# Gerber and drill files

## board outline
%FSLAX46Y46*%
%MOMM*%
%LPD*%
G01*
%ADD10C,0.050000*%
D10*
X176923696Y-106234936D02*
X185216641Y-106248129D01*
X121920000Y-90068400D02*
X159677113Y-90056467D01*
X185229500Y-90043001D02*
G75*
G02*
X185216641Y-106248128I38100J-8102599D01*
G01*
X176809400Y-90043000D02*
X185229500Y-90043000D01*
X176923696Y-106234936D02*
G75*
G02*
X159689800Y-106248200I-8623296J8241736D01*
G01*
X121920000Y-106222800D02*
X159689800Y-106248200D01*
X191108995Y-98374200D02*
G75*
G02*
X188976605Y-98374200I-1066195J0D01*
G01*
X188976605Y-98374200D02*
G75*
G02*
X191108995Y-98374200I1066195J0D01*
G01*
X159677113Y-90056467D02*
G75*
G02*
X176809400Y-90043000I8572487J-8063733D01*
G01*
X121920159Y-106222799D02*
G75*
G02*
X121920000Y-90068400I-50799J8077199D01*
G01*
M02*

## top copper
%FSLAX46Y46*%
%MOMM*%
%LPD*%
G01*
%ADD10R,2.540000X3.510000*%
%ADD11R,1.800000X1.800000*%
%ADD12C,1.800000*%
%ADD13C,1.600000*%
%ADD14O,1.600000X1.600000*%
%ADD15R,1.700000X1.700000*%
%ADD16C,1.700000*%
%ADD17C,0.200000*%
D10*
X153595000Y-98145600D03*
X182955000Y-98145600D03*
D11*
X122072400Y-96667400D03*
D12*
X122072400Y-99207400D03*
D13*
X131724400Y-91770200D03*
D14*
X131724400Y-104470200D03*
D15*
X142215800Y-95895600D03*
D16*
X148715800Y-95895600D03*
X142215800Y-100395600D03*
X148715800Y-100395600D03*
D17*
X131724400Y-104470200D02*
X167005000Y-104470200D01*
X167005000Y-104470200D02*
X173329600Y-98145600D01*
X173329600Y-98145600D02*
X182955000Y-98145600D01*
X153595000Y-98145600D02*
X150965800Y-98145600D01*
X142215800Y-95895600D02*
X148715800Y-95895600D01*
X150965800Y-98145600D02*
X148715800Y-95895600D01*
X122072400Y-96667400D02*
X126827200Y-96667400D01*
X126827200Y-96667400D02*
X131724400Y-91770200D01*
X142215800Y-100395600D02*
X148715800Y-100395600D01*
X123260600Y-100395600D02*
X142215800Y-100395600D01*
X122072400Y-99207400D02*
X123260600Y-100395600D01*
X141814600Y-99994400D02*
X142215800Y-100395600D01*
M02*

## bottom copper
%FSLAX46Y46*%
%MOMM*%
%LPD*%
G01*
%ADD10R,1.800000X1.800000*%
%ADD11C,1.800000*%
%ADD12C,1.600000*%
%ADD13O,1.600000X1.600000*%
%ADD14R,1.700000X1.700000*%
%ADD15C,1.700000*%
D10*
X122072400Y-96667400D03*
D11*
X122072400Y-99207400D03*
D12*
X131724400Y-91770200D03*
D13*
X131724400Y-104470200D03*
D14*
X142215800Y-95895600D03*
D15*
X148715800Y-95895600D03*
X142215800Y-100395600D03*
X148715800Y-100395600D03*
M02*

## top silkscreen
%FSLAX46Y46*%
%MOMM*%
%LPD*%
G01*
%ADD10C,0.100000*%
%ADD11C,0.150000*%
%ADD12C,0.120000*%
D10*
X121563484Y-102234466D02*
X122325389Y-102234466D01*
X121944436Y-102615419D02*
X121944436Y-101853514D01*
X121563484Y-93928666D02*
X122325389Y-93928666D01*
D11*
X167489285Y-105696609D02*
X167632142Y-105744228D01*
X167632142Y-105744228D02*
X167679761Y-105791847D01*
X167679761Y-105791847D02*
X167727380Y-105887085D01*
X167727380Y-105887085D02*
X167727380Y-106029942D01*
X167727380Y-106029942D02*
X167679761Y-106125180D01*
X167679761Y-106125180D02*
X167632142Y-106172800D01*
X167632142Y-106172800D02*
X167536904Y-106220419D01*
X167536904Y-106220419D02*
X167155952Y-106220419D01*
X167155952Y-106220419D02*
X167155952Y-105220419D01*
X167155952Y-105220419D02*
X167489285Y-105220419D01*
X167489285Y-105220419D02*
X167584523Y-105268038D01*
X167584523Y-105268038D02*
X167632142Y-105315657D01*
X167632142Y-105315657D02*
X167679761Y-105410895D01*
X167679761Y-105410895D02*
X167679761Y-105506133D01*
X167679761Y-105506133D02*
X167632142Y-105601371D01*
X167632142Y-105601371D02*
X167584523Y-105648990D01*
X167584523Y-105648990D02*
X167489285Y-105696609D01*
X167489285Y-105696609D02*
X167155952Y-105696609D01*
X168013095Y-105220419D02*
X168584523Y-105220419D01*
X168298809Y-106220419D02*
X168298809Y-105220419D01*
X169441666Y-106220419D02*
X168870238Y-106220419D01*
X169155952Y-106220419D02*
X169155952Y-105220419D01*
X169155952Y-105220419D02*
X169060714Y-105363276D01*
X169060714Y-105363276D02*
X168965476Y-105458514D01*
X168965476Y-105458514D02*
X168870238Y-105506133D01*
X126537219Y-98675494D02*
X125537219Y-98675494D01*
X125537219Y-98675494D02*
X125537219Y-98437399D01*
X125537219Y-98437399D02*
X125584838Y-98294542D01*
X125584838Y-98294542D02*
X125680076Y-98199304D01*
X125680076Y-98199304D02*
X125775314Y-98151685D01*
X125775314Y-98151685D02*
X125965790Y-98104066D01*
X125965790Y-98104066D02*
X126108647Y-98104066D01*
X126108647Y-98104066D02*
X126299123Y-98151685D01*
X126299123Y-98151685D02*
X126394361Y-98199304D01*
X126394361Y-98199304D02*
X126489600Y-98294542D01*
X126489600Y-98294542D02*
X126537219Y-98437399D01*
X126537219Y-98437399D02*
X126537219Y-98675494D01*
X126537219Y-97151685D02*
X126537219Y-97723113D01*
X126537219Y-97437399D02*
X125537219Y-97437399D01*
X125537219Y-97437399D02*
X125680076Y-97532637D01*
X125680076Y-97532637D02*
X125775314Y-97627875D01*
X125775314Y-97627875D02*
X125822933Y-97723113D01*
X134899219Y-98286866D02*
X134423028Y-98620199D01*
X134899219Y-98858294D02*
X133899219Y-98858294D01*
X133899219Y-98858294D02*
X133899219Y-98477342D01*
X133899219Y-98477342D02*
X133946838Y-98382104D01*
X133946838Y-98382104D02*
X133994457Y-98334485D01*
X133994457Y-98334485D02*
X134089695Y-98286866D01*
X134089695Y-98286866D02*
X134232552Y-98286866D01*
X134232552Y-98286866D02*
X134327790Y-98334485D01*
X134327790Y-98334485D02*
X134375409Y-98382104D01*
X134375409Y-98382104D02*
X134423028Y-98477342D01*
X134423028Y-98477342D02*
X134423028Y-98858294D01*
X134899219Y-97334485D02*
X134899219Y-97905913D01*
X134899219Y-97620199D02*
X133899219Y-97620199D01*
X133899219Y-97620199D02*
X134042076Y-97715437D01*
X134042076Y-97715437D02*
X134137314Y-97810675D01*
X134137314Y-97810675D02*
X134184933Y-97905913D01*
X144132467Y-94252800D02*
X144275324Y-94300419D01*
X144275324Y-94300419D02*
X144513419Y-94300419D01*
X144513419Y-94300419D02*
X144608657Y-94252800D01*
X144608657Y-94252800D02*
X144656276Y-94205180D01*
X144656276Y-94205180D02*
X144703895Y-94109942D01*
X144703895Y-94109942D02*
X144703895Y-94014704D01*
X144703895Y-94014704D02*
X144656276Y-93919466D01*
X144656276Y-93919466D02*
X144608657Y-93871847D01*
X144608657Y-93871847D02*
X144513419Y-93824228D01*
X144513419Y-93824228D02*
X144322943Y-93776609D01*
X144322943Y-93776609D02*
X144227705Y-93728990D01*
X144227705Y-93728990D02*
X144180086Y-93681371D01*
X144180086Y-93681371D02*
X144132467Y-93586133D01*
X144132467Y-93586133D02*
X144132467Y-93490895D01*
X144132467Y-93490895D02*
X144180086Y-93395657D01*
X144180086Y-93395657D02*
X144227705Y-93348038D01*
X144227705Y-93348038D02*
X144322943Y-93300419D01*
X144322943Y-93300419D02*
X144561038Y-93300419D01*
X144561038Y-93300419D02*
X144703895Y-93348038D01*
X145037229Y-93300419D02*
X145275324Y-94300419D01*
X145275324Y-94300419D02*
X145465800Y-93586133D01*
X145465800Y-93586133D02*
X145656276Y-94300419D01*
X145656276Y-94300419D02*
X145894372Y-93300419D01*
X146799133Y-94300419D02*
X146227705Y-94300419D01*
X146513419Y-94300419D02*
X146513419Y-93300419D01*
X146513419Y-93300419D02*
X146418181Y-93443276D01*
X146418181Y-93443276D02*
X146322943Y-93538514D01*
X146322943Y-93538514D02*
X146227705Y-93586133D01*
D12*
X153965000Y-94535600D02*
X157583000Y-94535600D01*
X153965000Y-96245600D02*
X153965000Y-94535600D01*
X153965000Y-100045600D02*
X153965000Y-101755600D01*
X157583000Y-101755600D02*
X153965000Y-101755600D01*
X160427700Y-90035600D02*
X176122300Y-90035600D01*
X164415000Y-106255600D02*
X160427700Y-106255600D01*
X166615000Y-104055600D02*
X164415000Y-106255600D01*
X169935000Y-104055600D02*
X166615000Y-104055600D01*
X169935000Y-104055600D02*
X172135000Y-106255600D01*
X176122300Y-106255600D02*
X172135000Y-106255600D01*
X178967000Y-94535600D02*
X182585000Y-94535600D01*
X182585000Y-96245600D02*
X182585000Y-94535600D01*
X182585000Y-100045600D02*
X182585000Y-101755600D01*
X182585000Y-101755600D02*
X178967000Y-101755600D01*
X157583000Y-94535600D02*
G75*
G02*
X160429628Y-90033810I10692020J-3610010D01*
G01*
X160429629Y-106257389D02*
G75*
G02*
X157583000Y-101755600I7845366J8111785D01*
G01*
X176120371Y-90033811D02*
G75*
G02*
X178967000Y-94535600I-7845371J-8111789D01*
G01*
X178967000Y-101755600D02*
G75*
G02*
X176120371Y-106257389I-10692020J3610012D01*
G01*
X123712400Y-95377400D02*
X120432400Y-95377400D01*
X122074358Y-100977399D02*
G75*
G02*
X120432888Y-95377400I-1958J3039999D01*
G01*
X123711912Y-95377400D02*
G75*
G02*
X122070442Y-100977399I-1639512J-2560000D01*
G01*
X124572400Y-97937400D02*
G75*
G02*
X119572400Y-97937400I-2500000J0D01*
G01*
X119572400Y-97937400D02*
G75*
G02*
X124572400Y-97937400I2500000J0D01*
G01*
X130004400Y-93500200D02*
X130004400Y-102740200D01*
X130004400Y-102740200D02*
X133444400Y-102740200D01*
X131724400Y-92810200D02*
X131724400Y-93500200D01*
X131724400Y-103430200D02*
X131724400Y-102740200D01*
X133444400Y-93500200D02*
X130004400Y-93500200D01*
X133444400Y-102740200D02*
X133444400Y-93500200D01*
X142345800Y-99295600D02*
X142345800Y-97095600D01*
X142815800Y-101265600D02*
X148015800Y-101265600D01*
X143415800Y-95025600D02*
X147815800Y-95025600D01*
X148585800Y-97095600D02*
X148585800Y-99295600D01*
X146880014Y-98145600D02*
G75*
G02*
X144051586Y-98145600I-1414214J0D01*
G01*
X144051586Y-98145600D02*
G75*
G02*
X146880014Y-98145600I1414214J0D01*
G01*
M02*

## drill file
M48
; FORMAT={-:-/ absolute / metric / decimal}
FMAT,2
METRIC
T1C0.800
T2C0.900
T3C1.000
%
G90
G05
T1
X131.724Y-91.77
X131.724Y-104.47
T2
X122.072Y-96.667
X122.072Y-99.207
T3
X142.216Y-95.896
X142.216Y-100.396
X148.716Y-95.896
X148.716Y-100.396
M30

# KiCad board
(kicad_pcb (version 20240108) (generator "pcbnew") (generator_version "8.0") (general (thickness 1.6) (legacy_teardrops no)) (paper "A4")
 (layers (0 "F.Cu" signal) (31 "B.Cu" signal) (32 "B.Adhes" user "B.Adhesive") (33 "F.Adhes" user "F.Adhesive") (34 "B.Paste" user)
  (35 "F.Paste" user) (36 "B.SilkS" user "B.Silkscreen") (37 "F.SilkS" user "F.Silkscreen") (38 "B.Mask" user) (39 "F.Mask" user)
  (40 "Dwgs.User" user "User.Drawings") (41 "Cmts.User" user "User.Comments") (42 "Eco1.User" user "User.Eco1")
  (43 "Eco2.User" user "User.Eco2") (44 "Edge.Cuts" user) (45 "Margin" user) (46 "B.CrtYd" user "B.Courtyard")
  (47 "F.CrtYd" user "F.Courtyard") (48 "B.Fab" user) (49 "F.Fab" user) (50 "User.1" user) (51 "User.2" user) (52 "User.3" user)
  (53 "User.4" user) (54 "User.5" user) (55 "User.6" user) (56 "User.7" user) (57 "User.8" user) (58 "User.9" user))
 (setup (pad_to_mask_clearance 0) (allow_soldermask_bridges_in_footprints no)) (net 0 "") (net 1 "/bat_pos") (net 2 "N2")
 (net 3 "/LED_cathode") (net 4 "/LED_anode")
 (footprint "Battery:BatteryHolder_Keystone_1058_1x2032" (layer "F.Cu") (at 168.275 98.1456)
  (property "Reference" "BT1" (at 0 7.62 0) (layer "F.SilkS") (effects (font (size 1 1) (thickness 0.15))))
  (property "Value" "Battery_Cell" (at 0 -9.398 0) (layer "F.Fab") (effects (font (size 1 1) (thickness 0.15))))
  (fp_line (start -14.31 -3.61) (end -10.692 -3.61) (stroke (width 0.12) (type solid)) (layer "F.SilkS"))
  (fp_line (start -14.31 -1.9) (end -14.31 -3.61) (stroke (width 0.12) (type solid)) (layer "F.SilkS"))
  (fp_line (start -14.31 1.9) (end -14.31 3.61) (stroke (width 0.12) (type solid)) (layer "F.SilkS"))
  (fp_line (start -10.692 3.61) (end -14.31 3.61) (stroke (width 0.12) (type solid)) (layer "F.SilkS"))
  (fp_line (start -7.8473 -8.11) (end 7.8473 -8.11) (stroke (width 0.12) (type solid)) (layer "F.SilkS"))
  (fp_line (start -3.86 8.11) (end -7.8473 8.11) (stroke (width 0.12) (type solid)) (layer "F.SilkS"))
  (fp_line (start -1.66 5.91) (end -3.86 8.11) (stroke (width 0.12) (type solid)) (layer "F.SilkS"))
  (fp_line (start 1.66 5.91) (end -1.66 5.91) (stroke (width 0.12) (type solid)) (layer "F.SilkS"))
  (fp_line (start 1.66 5.91) (end 3.86 8.11) (stroke (width 0.12) (type solid)) (layer "F.SilkS"))
  (fp_line (start 7.8473 8.11) (end 3.86 8.11) (stroke (width 0.12) (type solid)) (layer "F.SilkS"))
  (fp_line (start 10.692 -3.61) (end 14.31 -3.61) (stroke (width 0.12) (type solid)) (layer "F.SilkS"))
  (fp_line (start 14.31 -1.9) (end 14.31 -3.61) (stroke (width 0.12) (type solid)) (layer "F.SilkS"))
  (fp_line (start 14.31 1.9) (end 14.31 3.61) (stroke (width 0.12) (type solid)) (layer "F.SilkS"))
  (fp_line (start 14.31 3.61) (end 10.692 3.61) (stroke (width 0.12) (type solid)) (layer "F.SilkS"))
  (fp_arc (start -10.692 -3.61) (mid -9.538084 -6.031244) (end -7.845371 -8.111789) (stroke (width 0.12) (type solid)) (layer "F.SilkS"))
  (fp_arc (start -7.845371 8.111789) (mid -9.538085 6.031244) (end -10.692 3.61) (stroke (width 0.12) (type solid)) (layer "F.SilkS"))
  (fp_arc (start 7.845371 -8.111789) (mid 9.538085 -6.031244) (end 10.692 -3.61) (stroke (width 0.12) (type solid)) (layer "F.SilkS"))
  (fp_arc (start 10.692 3.61) (mid 9.538084 6.031244) (end 7.845371 8.111789) (stroke (width 0.12) (type solid)) (layer "F.SilkS"))
  (pad "1" smd rect (at -14.68 0) (size 2.54 3.51) (layers "F.Cu" "F.Paste" "F.Mask") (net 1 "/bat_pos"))
  (pad "2" smd rect (at 14.68 0) (size 2.54 3.51) (layers "F.Cu" "F.Paste" "F.Mask") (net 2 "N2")))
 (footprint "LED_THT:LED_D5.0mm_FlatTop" (layer "F.Cu") (at 122.0724 96.6674 -90)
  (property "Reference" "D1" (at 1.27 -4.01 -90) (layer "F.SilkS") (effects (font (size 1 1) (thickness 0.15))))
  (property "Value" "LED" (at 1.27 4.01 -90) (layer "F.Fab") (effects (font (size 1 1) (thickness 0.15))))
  (fp_line (start -1.29 -1.64) (end -1.29 1.64) (stroke (width 0.12) (type solid)) (layer "F.SilkS"))
  (fp_arc (start 4.309999 -0.001958) (mid 2.125106 2.917258) (end -1.29 1.639512) (stroke (width 0.12) (type solid)) (layer "F.SilkS"))
  (fp_arc (start -1.29 -1.639512) (mid 2.125106 -2.917258) (end 4.309999 0.001958) (stroke (width 0.12) (type solid)) (layer "F.SilkS"))
  (fp_circle (center 1.27 0) (end 3.77 0) (stroke (width 0.12) (type solid)) (fill none) (layer "F.SilkS"))
  (pad "1" thru_hole rect (at 0 0 270) (size 1.8 1.8) (drill 0.9) (layers "*.Cu" "*.Mask") (remove_unused_layers no) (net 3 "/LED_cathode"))
  (pad "2" thru_hole circle (at 2.54 0 270) (size 1.8 1.8) (drill 0.9) (layers "*.Cu" "*.Mask") (remove_unused_layers no)
   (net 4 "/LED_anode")))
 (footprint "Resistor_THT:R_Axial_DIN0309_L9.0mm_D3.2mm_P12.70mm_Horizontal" (layer "F.Cu") (at 131.7244 91.7702 -90)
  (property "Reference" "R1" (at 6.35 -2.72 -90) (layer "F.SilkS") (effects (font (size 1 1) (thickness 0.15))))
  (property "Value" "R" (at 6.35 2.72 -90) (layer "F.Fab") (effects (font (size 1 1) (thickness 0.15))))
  (fp_line (start 1.73 1.72) (end 10.97 1.72) (stroke (width 0.12) (type solid)) (layer "F.SilkS"))
  (fp_line (start 10.97 1.72) (end 10.97 -1.72) (stroke (width 0.12) (type solid)) (layer "F.SilkS"))
  (fp_line (start 1.04 0) (end 1.73 0) (stroke (width 0.12) (type solid)) (layer "F.SilkS"))
  (fp_line (start 11.66 0) (end 10.97 0) (stroke (width 0.12) (type solid)) (layer "F.SilkS"))
  (fp_line (start 1.73 -1.72) (end 1.73 1.72) (stroke (width 0.12) (type solid)) (layer "F.SilkS"))
  (fp_line (start 10.97 -1.72) (end 1.73 -1.72) (stroke (width 0.12) (type solid)) (layer "F.SilkS"))
  (pad "1" thru_hole circle (at 0 0 270) (size 1.6 1.6) (drill 0.8) (layers "*.Cu" "*.Mask") (remove_unused_layers no)
   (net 3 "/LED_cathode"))
  (pad "2" thru_hole oval (at 12.7 0 270) (size 1.6 1.6) (drill 0.8) (layers "*.Cu" "*.Mask") (remove_unused_layers no) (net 2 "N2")))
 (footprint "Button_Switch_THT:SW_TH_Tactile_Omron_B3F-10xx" (layer "F.Cu") (at 142.2158 95.8956)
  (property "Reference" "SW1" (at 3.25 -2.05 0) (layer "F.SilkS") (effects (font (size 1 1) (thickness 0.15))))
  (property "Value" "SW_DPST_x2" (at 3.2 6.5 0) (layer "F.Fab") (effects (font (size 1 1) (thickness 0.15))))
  (fp_line (start 0.13 3.4) (end 0.13 1.2) (stroke (width 0.12) (type solid)) (layer "F.SilkS"))
  (fp_line (start 0.6 5.37) (end 5.8 5.37) (stroke (width 0.12) (type solid)) (layer "F.SilkS"))
  (fp_line (start 1.2 -0.87) (end 5.6 -0.87) (stroke (width 0.12) (type solid)) (layer "F.SilkS"))
  (fp_line (start 6.37 1.2) (end 6.37 3.4) (stroke (width 0.12) (type solid)) (layer "F.SilkS"))
  (fp_circle (center 3.25 2.25) (end 4.25 3.25) (stroke (width 0.12) (type solid)) (fill none) (layer "F.SilkS"))
  (pad "1" thru_hole rect (at 0 0) (size 1.7 1.7) (drill 1) (layers "*.Cu" "*.Mask") (remove_unused_layers no) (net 1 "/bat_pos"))
  (pad "1" thru_hole circle (at 6.5 0) (size 1.7 1.7) (drill 1) (layers "*.Cu" "*.Mask") (remove_unused_layers no) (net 1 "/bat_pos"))
  (pad "2" thru_hole circle (at 0 4.5) (size 1.7 1.7) (drill 1) (layers "*.Cu" "*.Mask") (remove_unused_layers no) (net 4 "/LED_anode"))
  (pad "2" thru_hole circle (at 6.5 4.5) (size 1.7 1.7) (drill 1) (layers "*.Cu" "*.Mask") (remove_unused_layers no) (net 4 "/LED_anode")))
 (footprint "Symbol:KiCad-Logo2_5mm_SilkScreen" (layer "B.Cu") (at 168.3258 97.4852 180)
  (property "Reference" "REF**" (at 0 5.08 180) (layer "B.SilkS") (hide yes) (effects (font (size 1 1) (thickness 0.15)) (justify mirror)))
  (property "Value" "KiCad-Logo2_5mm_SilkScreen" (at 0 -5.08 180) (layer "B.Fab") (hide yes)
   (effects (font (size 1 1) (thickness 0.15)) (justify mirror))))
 (gr_line (start 176.923696 106.234936) (end 185.216641 106.248129) (stroke (width 0.05) (type default)) (layer "Edge.Cuts"))
 (gr_line (start 121.92 90.0684) (end 159.677113 90.056467) (stroke (width 0.05) (type default)) (layer "Edge.Cuts"))
 (gr_arc (start 185.2295 90.043001) (mid 193.370286 98.15203) (end 185.216641 106.248129) (stroke (width 0.05) (type default))
  (layer "Edge.Cuts"))
 (gr_line (start 176.8094 90.043) (end 185.2295 90.043) (stroke (width 0.05) (type default)) (layer "Edge.Cuts"))
 (gr_arc (start 176.923696 106.234936) (mid 168.30958 109.921627) (end 159.6898 106.2482) (stroke (width 0.05) (type default))
  (layer "Edge.Cuts"))
 (gr_line (start 121.92 106.2228) (end 159.6898 106.2482) (stroke (width 0.05) (type default)) (layer "Edge.Cuts"))
 (gr_circle (center 190.0428 98.3742) (end 190.2714 97.3328) (stroke (width 0.05) (type default)) (fill none) (layer "Edge.Cuts"))
 (gr_arc (start 159.677113 90.056467) (mid 168.240349 86.35112) (end 176.809399 90.043001) (stroke (width 0.05) (type default))
  (layer "Edge.Cuts"))
 (gr_arc (start 121.920159 106.222799) (mid 113.792 98.14568) (end 121.92 90.0684) (stroke (width 0.05) (type default)) (layer "Edge.Cuts"))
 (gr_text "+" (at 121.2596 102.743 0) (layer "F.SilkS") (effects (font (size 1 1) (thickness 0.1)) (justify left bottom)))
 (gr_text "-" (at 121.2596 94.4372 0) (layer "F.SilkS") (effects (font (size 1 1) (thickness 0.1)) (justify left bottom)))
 (segment (start 131.7244 104.4702) (end 167.005 104.4702) (width 0.2) (layer "F.Cu") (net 2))
 (segment (start 167.005 104.4702) (end 173.3296 98.1456) (width 0.2) (layer "F.Cu") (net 2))
 (segment (start 173.3296 98.1456) (end 182.955 98.1456) (width 0.2) (layer "F.Cu") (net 2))
 (segment (start 153.595 98.1456) (end 150.9658 98.1456) (width 0.2) (layer "F.Cu") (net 1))
 (segment (start 142.2158 95.8956) (end 148.7158 95.8956) (width 0.2) (layer "F.Cu") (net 1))
 (segment (start 150.9658 98.1456) (end 148.7158 95.8956) (width 0.2) (layer "F.Cu") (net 1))
 (segment (start 122.0724 96.6674) (end 126.8272 96.6674) (width 0.2) (layer "F.Cu") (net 3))
 (segment (start 126.8272 96.6674) (end 131.7244 91.7702) (width 0.2) (layer "F.Cu") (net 3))
 (segment (start 142.2158 100.3956) (end 148.7158 100.3956) (width 0.2) (layer "F.Cu") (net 4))
 (segment (start 123.2606 100.3956) (end 142.2158 100.3956) (width 0.2) (layer "F.Cu") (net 4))
 (segment (start 122.0724 99.2074) (end 123.2606 100.3956) (width 0.2) (layer "F.Cu") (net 4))
 (segment (start 141.8146 99.9944) (end 142.2158 100.3956) (width 0.2) (layer "F.Cu") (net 4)))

